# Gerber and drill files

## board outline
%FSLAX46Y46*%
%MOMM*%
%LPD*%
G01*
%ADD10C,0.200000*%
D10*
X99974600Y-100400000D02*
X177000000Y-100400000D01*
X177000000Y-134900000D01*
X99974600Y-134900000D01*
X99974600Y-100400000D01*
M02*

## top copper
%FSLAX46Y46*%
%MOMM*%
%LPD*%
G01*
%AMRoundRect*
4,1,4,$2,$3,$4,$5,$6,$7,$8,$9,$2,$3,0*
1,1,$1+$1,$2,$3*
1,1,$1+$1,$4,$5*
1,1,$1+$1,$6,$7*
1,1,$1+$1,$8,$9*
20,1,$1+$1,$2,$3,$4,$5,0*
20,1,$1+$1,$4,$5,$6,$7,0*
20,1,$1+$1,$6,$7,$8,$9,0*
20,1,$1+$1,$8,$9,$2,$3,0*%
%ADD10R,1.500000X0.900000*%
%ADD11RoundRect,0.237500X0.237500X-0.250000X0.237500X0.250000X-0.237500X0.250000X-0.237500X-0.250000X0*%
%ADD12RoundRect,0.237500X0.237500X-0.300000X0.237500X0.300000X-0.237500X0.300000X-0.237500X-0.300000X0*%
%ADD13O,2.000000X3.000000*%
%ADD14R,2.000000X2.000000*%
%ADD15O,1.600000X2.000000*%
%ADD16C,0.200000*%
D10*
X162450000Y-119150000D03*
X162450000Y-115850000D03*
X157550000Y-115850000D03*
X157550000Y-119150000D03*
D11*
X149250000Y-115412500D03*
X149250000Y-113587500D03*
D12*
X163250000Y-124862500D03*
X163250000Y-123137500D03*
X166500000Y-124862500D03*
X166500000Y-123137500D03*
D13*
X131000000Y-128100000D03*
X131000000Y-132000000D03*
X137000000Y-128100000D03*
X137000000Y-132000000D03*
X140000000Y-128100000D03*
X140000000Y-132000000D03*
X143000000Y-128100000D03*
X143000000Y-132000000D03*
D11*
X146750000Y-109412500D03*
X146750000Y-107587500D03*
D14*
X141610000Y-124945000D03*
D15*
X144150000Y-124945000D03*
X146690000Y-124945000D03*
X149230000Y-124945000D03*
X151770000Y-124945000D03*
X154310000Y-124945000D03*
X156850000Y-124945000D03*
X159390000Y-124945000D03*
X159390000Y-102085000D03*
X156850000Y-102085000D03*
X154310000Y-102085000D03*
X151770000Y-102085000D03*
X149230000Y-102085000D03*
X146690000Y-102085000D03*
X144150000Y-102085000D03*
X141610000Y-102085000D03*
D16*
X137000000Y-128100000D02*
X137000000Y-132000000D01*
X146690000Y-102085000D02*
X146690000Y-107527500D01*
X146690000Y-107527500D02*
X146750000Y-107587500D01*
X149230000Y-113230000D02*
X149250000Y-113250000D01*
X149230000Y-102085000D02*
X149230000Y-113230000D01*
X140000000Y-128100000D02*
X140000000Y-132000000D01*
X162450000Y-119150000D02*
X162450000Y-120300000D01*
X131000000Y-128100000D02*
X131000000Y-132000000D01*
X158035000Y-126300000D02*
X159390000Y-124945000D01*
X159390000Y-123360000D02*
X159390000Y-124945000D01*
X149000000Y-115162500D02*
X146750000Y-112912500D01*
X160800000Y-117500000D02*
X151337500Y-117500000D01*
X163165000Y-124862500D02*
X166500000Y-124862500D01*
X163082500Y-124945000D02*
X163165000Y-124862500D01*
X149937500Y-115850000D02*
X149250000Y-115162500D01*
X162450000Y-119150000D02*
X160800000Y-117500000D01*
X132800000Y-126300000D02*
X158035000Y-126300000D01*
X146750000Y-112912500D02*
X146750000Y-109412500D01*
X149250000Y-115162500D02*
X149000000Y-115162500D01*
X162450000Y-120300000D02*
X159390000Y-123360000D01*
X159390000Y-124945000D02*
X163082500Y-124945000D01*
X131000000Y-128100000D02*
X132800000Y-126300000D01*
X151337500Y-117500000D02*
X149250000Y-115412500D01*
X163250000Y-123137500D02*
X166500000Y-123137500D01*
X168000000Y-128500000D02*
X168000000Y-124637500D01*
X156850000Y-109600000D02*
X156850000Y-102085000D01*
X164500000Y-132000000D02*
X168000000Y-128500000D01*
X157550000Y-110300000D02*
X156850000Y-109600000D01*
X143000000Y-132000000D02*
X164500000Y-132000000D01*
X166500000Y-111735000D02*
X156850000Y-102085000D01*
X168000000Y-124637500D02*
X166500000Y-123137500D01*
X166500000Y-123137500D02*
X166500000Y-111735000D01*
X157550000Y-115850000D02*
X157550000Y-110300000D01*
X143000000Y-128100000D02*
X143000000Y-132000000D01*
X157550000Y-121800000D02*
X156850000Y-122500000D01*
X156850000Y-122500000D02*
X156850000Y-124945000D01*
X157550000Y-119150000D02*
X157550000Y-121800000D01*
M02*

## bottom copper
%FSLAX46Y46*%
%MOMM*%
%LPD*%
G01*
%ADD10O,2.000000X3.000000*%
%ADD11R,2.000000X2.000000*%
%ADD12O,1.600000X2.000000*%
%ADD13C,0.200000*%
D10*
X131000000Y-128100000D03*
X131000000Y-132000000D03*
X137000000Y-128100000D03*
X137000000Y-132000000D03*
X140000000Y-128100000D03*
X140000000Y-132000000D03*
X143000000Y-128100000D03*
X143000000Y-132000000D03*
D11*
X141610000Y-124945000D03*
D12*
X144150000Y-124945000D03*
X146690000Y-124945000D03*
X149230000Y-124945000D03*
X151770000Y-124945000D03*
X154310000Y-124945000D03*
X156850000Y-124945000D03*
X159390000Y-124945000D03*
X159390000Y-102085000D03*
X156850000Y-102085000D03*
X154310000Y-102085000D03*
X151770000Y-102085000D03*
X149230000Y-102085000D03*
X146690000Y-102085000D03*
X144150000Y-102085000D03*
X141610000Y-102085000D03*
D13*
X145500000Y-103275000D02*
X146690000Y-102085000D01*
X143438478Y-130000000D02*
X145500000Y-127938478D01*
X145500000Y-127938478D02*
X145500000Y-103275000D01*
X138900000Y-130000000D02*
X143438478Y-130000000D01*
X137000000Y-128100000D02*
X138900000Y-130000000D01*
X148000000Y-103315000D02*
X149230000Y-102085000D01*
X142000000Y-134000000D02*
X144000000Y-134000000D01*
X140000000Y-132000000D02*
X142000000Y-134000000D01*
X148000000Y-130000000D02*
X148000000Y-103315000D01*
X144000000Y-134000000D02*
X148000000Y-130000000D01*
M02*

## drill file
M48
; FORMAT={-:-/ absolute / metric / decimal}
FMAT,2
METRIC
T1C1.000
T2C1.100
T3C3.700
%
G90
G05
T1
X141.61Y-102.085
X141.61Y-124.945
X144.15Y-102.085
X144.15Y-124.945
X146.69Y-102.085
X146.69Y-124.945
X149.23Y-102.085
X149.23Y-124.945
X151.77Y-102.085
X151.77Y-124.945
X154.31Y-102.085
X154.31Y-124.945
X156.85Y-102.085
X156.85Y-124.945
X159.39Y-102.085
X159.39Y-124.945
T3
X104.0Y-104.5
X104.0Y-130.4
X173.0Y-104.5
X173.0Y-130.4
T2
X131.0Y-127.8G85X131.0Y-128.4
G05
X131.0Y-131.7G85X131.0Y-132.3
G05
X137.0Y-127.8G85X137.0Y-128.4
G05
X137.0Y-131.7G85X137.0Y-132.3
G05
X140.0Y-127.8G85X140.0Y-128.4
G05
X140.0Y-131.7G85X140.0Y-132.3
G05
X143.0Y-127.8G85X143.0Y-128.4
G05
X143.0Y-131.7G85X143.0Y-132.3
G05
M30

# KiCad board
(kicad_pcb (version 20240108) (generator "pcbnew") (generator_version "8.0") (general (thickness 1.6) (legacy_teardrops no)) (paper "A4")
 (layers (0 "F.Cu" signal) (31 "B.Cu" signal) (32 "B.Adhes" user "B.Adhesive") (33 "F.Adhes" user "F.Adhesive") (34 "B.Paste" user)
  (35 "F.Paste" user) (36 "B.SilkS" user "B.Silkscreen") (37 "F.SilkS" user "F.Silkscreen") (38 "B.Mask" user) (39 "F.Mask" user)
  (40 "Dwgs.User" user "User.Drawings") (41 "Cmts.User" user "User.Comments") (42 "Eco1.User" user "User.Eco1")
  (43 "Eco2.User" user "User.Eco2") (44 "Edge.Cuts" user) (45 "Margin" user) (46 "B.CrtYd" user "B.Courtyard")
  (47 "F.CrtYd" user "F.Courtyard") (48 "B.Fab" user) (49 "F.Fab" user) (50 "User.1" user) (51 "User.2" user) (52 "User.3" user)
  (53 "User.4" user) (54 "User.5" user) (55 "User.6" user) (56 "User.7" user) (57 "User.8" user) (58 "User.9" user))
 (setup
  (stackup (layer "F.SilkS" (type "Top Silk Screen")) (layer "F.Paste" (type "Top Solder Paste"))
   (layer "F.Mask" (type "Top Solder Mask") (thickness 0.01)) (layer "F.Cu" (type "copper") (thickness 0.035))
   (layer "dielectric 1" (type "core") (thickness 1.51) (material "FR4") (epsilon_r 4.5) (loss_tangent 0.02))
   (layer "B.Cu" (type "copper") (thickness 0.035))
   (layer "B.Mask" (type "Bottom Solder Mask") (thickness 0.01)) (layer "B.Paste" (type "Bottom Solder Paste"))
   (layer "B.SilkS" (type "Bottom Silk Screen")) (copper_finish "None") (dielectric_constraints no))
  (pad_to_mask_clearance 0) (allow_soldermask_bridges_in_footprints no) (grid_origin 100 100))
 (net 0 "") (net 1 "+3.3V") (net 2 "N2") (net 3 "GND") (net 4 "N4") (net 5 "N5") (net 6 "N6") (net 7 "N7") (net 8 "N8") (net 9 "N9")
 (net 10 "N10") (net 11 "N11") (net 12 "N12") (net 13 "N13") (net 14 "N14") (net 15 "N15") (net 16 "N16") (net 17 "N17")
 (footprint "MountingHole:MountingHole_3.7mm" (layer "F.Cu") (at 173 130.4)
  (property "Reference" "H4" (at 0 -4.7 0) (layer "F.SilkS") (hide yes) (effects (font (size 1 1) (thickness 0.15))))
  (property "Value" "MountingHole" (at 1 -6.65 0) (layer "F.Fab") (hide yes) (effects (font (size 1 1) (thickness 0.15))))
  (pad "" np_thru_hole circle (at 0 0) (size 3.7 3.7) (drill 3.7) (layers "*.Cu" "*.Mask")))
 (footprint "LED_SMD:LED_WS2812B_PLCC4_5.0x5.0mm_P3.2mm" (layer "F.Cu") (at 160 117.5 180)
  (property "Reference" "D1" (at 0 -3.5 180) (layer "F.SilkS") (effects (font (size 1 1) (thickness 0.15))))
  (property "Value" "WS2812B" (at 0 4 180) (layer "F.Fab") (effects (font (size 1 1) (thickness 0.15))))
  (pad "1" smd rect (at -2.45 -1.65 180) (size 1.5 0.9) (layers "F.Cu" "F.Paste" "F.Mask") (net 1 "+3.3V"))
  (pad "2" smd rect (at -2.45 1.65 180) (size 1.5 0.9) (layers "F.Cu" "F.Paste" "F.Mask") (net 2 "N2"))
  (pad "3" smd rect (at 2.45 1.65 180) (size 1.5 0.9) (layers "F.Cu" "F.Paste" "F.Mask") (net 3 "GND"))
  (pad "4" smd rect (at 2.45 -1.65 180) (size 1.5 0.9) (layers "F.Cu" "F.Paste" "F.Mask") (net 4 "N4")))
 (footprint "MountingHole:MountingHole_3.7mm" (layer "F.Cu") (at 173 104.5)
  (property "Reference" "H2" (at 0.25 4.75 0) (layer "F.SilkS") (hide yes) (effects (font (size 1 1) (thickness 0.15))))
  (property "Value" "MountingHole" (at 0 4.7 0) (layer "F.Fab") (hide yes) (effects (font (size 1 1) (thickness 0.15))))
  (pad "" np_thru_hole circle (at 0 0) (size 3.7 3.7) (drill 3.7) (layers "*.Cu" "*.Mask")))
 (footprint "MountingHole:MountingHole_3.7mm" (layer "F.Cu") (at 104 130.4)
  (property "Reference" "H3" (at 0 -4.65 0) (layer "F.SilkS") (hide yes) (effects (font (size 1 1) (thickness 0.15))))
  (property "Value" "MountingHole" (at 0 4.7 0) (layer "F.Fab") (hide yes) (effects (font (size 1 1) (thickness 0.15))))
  (pad "" np_thru_hole circle (at 0 0) (size 3.7 3.7) (drill 3.7) (layers "*.Cu" "*.Mask")))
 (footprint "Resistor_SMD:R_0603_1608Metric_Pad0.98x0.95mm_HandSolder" (layer "F.Cu") (at 149.25 114.5 90)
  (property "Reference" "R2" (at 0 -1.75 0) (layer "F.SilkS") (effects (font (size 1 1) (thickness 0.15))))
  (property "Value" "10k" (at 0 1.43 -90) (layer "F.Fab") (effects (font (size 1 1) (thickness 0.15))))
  (pad "1" smd roundrect (at -0.9125 0 90) (size 0.975 0.95) (layers "F.Cu" "F.Paste" "F.Mask") (roundrect_rratio 0.25) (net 1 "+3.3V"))
  (pad "2" smd roundrect (at 0.9125 0 90) (size 0.975 0.95) (layers "F.Cu" "F.Paste" "F.Mask") (roundrect_rratio 0.25) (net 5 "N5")))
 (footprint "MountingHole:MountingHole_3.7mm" (layer "F.Cu") (at 104 104.5)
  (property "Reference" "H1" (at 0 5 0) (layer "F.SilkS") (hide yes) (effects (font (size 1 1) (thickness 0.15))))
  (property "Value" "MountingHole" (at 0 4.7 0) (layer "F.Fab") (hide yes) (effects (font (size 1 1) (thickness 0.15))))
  (pad "" np_thru_hole circle (at 0 0) (size 3.7 3.7) (drill 3.7) (layers "*.Cu" "*.Mask")))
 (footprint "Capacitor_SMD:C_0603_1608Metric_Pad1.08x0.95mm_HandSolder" (layer "F.Cu") (at 163.25 124 90)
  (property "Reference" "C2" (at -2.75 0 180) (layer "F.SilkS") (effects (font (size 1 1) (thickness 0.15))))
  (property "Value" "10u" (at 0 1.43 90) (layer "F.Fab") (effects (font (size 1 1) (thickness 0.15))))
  (pad "1" smd roundrect (at -0.8625 0 90) (size 1.075 0.95) (layers "F.Cu" "F.Paste" "F.Mask") (roundrect_rratio 0.25) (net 1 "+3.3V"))
  (pad "2" smd roundrect (at 0.8625 0 90) (size 1.075 0.95) (layers "F.Cu" "F.Paste" "F.Mask") (roundrect_rratio 0.25) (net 3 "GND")))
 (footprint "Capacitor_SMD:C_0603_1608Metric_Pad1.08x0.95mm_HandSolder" (layer "F.Cu") (at 166.5 124 90)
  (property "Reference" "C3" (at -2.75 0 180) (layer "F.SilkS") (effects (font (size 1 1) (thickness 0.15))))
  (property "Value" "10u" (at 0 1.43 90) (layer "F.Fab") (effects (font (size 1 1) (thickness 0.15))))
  (pad "1" smd roundrect (at -0.8625 0 90) (size 1.075 0.95) (layers "F.Cu" "F.Paste" "F.Mask") (roundrect_rratio 0.25) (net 1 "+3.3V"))
  (pad "2" smd roundrect (at 0.8625 0 90) (size 1.075 0.95) (layers "F.Cu" "F.Paste" "F.Mask") (roundrect_rratio 0.25) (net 3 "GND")))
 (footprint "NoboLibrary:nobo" (layer "F.Cu") (at 131 132)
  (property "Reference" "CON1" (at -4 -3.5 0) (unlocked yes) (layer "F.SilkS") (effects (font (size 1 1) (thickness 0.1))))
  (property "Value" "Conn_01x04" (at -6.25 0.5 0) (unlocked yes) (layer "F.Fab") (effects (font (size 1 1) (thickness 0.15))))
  (pad "1" thru_hole oval (at 0 -3.9) (size 2 3) (drill oval 1.1 1.7) (layers "*.Cu" "*.Mask") (remove_unused_layers no) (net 1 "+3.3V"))
  (pad "1" thru_hole oval (at 0 0) (size 2 3) (drill oval 1.1 1.7) (layers "*.Cu" "*.Mask") (remove_unused_layers no) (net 1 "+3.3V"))
  (pad "2" thru_hole oval (at 6 -3.9) (size 2 3) (drill oval 1.1 1.7) (layers "*.Cu" "*.Mask") (remove_unused_layers no) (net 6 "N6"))
  (pad "2" thru_hole oval (at 6 0) (size 2 3) (drill oval 1.1 1.7) (layers "*.Cu" "*.Mask") (remove_unused_layers no) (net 6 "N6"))
  (pad "3" thru_hole oval (at 9 -3.9) (size 2 3) (drill oval 1.1 1.7) (layers "*.Cu" "*.Mask") (remove_unused_layers no) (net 5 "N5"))
  (pad "3" thru_hole oval (at 9 0) (size 2 3) (drill oval 1.1 1.7) (layers "*.Cu" "*.Mask") (remove_unused_layers no) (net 5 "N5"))
  (pad "4" thru_hole oval (at 12 -3.9) (size 2 3) (drill oval 1.1 1.7) (layers "*.Cu" "*.Mask") (remove_unused_layers no) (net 3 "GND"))
  (pad "4" thru_hole oval (at 12 0) (size 2 3) (drill oval 1.1 1.7) (layers "*.Cu" "*.Mask") (remove_unused_layers no) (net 3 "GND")))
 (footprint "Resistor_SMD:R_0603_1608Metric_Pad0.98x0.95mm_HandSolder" (layer "F.Cu") (at 146.75 108.5 90)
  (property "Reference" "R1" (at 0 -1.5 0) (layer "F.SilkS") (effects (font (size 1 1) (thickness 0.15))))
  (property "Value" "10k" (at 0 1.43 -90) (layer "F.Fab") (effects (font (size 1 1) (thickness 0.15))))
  (pad "1" smd roundrect (at -0.9125 0 90) (size 0.975 0.95) (layers "F.Cu" "F.Paste" "F.Mask") (roundrect_rratio 0.25) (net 1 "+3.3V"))
  (pad "2" smd roundrect (at 0.9125 0 90) (size 0.975 0.95) (layers "F.Cu" "F.Paste" "F.Mask") (roundrect_rratio 0.25) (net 6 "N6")))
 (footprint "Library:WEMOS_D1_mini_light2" (layer "B.Cu") (at 141.61 103.145 -90)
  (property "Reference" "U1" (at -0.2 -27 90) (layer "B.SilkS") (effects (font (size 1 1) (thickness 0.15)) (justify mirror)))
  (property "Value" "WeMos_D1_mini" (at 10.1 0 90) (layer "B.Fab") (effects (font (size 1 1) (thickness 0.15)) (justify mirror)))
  (pad "1" thru_hole rect (at 21.8 0 270) (size 2 2) (drill 1) (layers "*.Cu" "*.Mask") (remove_unused_layers no) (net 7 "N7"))
  (pad "2" thru_hole oval (at 21.8 -2.54 270) (size 2 1.6) (drill 1) (layers "*.Cu" "*.Mask") (remove_unused_layers no) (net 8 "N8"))
  (pad "3" thru_hole oval (at 21.8 -5.08 270) (size 2 1.6) (drill 1) (layers "*.Cu" "*.Mask") (remove_unused_layers no) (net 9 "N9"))
  (pad "4" thru_hole oval (at 21.8 -7.62 270) (size 2 1.6) (drill 1) (layers "*.Cu" "*.Mask") (remove_unused_layers no) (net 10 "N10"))
  (pad "5" thru_hole oval (at 21.8 -10.16 270) (size 2 1.6) (drill 1) (layers "*.Cu" "*.Mask") (remove_unused_layers no) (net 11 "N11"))
  (pad "6" thru_hole oval (at 21.8 -12.7 270) (size 2 1.6) (drill 1) (layers "*.Cu" "*.Mask") (remove_unused_layers no) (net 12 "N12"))
  (pad "7" thru_hole oval (at 21.8 -15.24 270) (size 2 1.6) (drill 1) (layers "*.Cu" "*.Mask") (remove_unused_layers no) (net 4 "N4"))
  (pad "8" thru_hole oval (at 21.8 -17.78 270) (size 2 1.6) (drill 1) (layers "*.Cu" "*.Mask") (remove_unused_layers no) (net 1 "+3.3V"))
  (pad "9" thru_hole oval (at -1.06 -17.78 270) (size 2 1.6) (drill 1) (layers "*.Cu" "*.Mask") (remove_unused_layers no) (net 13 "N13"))
  (pad "10" thru_hole oval (at -1.06 -15.24 270) (size 2 1.6) (drill 1) (layers "*.Cu" "*.Mask") (remove_unused_layers no) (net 3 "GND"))
  (pad "11" thru_hole oval (at -1.06 -12.7 270) (size 2 1.6) (drill 1) (layers "*.Cu" "*.Mask") (remove_unused_layers no) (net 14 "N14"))
  (pad "12" thru_hole oval (at -1.06 -10.16 270) (size 2 1.6) (drill 1) (layers "*.Cu" "*.Mask") (remove_unused_layers no) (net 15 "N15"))
  (pad "13" thru_hole oval (at -1.06 -7.62 270) (size 2 1.6) (drill 1) (layers "*.Cu" "*.Mask") (remove_unused_layers no) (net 5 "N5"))
  (pad "14" thru_hole oval (at -1.06 -5.08 270) (size 2 1.6) (drill 1) (layers "*.Cu" "*.Mask") (remove_unused_layers no) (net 6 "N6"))
  (pad "15" thru_hole oval (at -1.06 -2.54 270) (size 2 1.6) (drill 1) (layers "*.Cu" "*.Mask") (remove_unused_layers no) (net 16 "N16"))
  (pad "16" thru_hole oval (at -1.06 0 270) (size 2 1.6) (drill 1) (layers "*.Cu" "*.Mask") (remove_unused_layers no) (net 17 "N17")))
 (gr_rect (start 99.9746 100.4) (end 177 134.9) (stroke (width 0.2) (type default)) (fill none) (layer "Edge.Cuts"))
 (segment (start 137 128.1) (end 137 132) (width 0.2) (layer "F.Cu") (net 6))
 (segment (start 146.69 102.085) (end 146.69 107.5275) (width 0.2) (layer "F.Cu") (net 6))
 (segment (start 146.69 107.5275) (end 146.75 107.5875) (width 0.2) (layer "F.Cu") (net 6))
 (segment (start 145.5 103.275) (end 146.69 102.085) (width 0.2) (layer "B.Cu") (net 6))
 (segment (start 143.438478 130) (end 145.5 127.938478) (width 0.2) (layer "B.Cu") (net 6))
 (segment (start 145.5 127.938478) (end 145.5 103.275) (width 0.2) (layer "B.Cu") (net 6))
 (segment (start 138.9 130) (end 143.438478 130) (width 0.2) (layer "B.Cu") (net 6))
 (segment (start 137 128.1) (end 138.9 130) (width 0.2) (layer "B.Cu") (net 6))
 (segment (start 149.23 113.23) (end 149.25 113.25) (width 0.2) (layer "F.Cu") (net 5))
 (segment (start 149.23 102.085) (end 149.23 113.23) (width 0.2) (layer "F.Cu") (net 5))
 (segment (start 140 128.1) (end 140 132) (width 0.2) (layer "F.Cu") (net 5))
 (segment (start 148 103.315) (end 149.23 102.085) (width 0.2) (layer "B.Cu") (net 5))
 (segment (start 142 134) (end 144 134) (width 0.2) (layer "B.Cu") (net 5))
 (segment (start 140 132) (end 142 134) (width 0.2) (layer "B.Cu") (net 5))
 (segment (start 148 130) (end 148 103.315) (width 0.2) (layer "B.Cu") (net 5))
 (segment (start 144 134) (end 148 130) (width 0.2) (layer "B.Cu") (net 5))
 (segment (start 162.45 119.15) (end 162.45 120.3) (width 0.2) (layer "F.Cu") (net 1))
 (segment (start 131 128.1) (end 131 132) (width 0.2) (layer "F.Cu") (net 1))
 (segment (start 158.035 126.3) (end 159.39 124.945) (width 0.2) (layer "F.Cu") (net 1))
 (segment (start 159.39 123.36) (end 159.39 124.945) (width 0.2) (layer "F.Cu") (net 1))
 (segment (start 149 115.1625) (end 146.75 112.9125) (width 0.2) (layer "F.Cu") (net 1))
 (segment (start 160.8 117.5) (end 151.3375 117.5) (width 0.2) (layer "F.Cu") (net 1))
 (segment (start 163.165 124.8625) (end 166.5 124.8625) (width 0.2) (layer "F.Cu") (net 1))
 (segment (start 163.0825 124.945) (end 163.165 124.8625) (width 0.2) (layer "F.Cu") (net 1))
 (segment (start 149.9375 115.85) (end 149.25 115.1625) (width 0.2) (layer "F.Cu") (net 1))
 (segment (start 162.45 119.15) (end 160.8 117.5) (width 0.2) (layer "F.Cu") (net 1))
 (segment (start 132.8 126.3) (end 158.035 126.3) (width 0.2) (layer "F.Cu") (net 1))
 (segment (start 146.75 112.9125) (end 146.75 109.4125) (width 0.2) (layer "F.Cu") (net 1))
 (segment (start 149.25 115.1625) (end 149 115.1625) (width 0.2) (layer "F.Cu") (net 1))
 (segment (start 162.45 120.3) (end 159.39 123.36) (width 0.2) (layer "F.Cu") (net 1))
 (segment (start 159.39 124.945) (end 163.0825 124.945) (width 0.2) (layer "F.Cu") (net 1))
 (segment (start 131 128.1) (end 132.8 126.3) (width 0.2) (layer "F.Cu") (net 1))
 (segment (start 151.3375 117.5) (end 149.25 115.4125) (width 0.2) (layer "F.Cu") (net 1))
 (segment (start 163.25 123.1375) (end 166.5 123.1375) (width 0.2) (layer "F.Cu") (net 3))
 (segment (start 168 128.5) (end 168 124.6375) (width 0.2) (layer "F.Cu") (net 3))
 (segment (start 156.85 109.6) (end 156.85 102.085) (width 0.2) (layer "F.Cu") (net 3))
 (segment (start 164.5 132) (end 168 128.5) (width 0.2) (layer "F.Cu") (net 3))
 (segment (start 157.55 110.3) (end 156.85 109.6) (width 0.2) (layer "F.Cu") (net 3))
 (segment (start 143 132) (end 164.5 132) (width 0.2) (layer "F.Cu") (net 3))
 (segment (start 166.5 111.735) (end 156.85 102.085) (width 0.2) (layer "F.Cu") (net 3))
 (segment (start 168 124.6375) (end 166.5 123.1375) (width 0.2) (layer "F.Cu") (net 3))
 (segment (start 166.5 123.1375) (end 166.5 111.735) (width 0.2) (layer "F.Cu") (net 3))
 (segment (start 157.55 115.85) (end 157.55 110.3) (width 0.2) (layer "F.Cu") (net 3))
 (segment (start 143 128.1) (end 143 132) (width 0.2) (layer "F.Cu") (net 3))
 (segment (start 157.55 121.8) (end 156.85 122.5) (width 0.2) (layer "F.Cu") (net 4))
 (segment (start 156.85 122.5) (end 156.85 124.945) (width 0.2) (layer "F.Cu") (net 4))
 (segment (start 157.55 119.15) (end 157.55 121.8) (width 0.2) (layer "F.Cu") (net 4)))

